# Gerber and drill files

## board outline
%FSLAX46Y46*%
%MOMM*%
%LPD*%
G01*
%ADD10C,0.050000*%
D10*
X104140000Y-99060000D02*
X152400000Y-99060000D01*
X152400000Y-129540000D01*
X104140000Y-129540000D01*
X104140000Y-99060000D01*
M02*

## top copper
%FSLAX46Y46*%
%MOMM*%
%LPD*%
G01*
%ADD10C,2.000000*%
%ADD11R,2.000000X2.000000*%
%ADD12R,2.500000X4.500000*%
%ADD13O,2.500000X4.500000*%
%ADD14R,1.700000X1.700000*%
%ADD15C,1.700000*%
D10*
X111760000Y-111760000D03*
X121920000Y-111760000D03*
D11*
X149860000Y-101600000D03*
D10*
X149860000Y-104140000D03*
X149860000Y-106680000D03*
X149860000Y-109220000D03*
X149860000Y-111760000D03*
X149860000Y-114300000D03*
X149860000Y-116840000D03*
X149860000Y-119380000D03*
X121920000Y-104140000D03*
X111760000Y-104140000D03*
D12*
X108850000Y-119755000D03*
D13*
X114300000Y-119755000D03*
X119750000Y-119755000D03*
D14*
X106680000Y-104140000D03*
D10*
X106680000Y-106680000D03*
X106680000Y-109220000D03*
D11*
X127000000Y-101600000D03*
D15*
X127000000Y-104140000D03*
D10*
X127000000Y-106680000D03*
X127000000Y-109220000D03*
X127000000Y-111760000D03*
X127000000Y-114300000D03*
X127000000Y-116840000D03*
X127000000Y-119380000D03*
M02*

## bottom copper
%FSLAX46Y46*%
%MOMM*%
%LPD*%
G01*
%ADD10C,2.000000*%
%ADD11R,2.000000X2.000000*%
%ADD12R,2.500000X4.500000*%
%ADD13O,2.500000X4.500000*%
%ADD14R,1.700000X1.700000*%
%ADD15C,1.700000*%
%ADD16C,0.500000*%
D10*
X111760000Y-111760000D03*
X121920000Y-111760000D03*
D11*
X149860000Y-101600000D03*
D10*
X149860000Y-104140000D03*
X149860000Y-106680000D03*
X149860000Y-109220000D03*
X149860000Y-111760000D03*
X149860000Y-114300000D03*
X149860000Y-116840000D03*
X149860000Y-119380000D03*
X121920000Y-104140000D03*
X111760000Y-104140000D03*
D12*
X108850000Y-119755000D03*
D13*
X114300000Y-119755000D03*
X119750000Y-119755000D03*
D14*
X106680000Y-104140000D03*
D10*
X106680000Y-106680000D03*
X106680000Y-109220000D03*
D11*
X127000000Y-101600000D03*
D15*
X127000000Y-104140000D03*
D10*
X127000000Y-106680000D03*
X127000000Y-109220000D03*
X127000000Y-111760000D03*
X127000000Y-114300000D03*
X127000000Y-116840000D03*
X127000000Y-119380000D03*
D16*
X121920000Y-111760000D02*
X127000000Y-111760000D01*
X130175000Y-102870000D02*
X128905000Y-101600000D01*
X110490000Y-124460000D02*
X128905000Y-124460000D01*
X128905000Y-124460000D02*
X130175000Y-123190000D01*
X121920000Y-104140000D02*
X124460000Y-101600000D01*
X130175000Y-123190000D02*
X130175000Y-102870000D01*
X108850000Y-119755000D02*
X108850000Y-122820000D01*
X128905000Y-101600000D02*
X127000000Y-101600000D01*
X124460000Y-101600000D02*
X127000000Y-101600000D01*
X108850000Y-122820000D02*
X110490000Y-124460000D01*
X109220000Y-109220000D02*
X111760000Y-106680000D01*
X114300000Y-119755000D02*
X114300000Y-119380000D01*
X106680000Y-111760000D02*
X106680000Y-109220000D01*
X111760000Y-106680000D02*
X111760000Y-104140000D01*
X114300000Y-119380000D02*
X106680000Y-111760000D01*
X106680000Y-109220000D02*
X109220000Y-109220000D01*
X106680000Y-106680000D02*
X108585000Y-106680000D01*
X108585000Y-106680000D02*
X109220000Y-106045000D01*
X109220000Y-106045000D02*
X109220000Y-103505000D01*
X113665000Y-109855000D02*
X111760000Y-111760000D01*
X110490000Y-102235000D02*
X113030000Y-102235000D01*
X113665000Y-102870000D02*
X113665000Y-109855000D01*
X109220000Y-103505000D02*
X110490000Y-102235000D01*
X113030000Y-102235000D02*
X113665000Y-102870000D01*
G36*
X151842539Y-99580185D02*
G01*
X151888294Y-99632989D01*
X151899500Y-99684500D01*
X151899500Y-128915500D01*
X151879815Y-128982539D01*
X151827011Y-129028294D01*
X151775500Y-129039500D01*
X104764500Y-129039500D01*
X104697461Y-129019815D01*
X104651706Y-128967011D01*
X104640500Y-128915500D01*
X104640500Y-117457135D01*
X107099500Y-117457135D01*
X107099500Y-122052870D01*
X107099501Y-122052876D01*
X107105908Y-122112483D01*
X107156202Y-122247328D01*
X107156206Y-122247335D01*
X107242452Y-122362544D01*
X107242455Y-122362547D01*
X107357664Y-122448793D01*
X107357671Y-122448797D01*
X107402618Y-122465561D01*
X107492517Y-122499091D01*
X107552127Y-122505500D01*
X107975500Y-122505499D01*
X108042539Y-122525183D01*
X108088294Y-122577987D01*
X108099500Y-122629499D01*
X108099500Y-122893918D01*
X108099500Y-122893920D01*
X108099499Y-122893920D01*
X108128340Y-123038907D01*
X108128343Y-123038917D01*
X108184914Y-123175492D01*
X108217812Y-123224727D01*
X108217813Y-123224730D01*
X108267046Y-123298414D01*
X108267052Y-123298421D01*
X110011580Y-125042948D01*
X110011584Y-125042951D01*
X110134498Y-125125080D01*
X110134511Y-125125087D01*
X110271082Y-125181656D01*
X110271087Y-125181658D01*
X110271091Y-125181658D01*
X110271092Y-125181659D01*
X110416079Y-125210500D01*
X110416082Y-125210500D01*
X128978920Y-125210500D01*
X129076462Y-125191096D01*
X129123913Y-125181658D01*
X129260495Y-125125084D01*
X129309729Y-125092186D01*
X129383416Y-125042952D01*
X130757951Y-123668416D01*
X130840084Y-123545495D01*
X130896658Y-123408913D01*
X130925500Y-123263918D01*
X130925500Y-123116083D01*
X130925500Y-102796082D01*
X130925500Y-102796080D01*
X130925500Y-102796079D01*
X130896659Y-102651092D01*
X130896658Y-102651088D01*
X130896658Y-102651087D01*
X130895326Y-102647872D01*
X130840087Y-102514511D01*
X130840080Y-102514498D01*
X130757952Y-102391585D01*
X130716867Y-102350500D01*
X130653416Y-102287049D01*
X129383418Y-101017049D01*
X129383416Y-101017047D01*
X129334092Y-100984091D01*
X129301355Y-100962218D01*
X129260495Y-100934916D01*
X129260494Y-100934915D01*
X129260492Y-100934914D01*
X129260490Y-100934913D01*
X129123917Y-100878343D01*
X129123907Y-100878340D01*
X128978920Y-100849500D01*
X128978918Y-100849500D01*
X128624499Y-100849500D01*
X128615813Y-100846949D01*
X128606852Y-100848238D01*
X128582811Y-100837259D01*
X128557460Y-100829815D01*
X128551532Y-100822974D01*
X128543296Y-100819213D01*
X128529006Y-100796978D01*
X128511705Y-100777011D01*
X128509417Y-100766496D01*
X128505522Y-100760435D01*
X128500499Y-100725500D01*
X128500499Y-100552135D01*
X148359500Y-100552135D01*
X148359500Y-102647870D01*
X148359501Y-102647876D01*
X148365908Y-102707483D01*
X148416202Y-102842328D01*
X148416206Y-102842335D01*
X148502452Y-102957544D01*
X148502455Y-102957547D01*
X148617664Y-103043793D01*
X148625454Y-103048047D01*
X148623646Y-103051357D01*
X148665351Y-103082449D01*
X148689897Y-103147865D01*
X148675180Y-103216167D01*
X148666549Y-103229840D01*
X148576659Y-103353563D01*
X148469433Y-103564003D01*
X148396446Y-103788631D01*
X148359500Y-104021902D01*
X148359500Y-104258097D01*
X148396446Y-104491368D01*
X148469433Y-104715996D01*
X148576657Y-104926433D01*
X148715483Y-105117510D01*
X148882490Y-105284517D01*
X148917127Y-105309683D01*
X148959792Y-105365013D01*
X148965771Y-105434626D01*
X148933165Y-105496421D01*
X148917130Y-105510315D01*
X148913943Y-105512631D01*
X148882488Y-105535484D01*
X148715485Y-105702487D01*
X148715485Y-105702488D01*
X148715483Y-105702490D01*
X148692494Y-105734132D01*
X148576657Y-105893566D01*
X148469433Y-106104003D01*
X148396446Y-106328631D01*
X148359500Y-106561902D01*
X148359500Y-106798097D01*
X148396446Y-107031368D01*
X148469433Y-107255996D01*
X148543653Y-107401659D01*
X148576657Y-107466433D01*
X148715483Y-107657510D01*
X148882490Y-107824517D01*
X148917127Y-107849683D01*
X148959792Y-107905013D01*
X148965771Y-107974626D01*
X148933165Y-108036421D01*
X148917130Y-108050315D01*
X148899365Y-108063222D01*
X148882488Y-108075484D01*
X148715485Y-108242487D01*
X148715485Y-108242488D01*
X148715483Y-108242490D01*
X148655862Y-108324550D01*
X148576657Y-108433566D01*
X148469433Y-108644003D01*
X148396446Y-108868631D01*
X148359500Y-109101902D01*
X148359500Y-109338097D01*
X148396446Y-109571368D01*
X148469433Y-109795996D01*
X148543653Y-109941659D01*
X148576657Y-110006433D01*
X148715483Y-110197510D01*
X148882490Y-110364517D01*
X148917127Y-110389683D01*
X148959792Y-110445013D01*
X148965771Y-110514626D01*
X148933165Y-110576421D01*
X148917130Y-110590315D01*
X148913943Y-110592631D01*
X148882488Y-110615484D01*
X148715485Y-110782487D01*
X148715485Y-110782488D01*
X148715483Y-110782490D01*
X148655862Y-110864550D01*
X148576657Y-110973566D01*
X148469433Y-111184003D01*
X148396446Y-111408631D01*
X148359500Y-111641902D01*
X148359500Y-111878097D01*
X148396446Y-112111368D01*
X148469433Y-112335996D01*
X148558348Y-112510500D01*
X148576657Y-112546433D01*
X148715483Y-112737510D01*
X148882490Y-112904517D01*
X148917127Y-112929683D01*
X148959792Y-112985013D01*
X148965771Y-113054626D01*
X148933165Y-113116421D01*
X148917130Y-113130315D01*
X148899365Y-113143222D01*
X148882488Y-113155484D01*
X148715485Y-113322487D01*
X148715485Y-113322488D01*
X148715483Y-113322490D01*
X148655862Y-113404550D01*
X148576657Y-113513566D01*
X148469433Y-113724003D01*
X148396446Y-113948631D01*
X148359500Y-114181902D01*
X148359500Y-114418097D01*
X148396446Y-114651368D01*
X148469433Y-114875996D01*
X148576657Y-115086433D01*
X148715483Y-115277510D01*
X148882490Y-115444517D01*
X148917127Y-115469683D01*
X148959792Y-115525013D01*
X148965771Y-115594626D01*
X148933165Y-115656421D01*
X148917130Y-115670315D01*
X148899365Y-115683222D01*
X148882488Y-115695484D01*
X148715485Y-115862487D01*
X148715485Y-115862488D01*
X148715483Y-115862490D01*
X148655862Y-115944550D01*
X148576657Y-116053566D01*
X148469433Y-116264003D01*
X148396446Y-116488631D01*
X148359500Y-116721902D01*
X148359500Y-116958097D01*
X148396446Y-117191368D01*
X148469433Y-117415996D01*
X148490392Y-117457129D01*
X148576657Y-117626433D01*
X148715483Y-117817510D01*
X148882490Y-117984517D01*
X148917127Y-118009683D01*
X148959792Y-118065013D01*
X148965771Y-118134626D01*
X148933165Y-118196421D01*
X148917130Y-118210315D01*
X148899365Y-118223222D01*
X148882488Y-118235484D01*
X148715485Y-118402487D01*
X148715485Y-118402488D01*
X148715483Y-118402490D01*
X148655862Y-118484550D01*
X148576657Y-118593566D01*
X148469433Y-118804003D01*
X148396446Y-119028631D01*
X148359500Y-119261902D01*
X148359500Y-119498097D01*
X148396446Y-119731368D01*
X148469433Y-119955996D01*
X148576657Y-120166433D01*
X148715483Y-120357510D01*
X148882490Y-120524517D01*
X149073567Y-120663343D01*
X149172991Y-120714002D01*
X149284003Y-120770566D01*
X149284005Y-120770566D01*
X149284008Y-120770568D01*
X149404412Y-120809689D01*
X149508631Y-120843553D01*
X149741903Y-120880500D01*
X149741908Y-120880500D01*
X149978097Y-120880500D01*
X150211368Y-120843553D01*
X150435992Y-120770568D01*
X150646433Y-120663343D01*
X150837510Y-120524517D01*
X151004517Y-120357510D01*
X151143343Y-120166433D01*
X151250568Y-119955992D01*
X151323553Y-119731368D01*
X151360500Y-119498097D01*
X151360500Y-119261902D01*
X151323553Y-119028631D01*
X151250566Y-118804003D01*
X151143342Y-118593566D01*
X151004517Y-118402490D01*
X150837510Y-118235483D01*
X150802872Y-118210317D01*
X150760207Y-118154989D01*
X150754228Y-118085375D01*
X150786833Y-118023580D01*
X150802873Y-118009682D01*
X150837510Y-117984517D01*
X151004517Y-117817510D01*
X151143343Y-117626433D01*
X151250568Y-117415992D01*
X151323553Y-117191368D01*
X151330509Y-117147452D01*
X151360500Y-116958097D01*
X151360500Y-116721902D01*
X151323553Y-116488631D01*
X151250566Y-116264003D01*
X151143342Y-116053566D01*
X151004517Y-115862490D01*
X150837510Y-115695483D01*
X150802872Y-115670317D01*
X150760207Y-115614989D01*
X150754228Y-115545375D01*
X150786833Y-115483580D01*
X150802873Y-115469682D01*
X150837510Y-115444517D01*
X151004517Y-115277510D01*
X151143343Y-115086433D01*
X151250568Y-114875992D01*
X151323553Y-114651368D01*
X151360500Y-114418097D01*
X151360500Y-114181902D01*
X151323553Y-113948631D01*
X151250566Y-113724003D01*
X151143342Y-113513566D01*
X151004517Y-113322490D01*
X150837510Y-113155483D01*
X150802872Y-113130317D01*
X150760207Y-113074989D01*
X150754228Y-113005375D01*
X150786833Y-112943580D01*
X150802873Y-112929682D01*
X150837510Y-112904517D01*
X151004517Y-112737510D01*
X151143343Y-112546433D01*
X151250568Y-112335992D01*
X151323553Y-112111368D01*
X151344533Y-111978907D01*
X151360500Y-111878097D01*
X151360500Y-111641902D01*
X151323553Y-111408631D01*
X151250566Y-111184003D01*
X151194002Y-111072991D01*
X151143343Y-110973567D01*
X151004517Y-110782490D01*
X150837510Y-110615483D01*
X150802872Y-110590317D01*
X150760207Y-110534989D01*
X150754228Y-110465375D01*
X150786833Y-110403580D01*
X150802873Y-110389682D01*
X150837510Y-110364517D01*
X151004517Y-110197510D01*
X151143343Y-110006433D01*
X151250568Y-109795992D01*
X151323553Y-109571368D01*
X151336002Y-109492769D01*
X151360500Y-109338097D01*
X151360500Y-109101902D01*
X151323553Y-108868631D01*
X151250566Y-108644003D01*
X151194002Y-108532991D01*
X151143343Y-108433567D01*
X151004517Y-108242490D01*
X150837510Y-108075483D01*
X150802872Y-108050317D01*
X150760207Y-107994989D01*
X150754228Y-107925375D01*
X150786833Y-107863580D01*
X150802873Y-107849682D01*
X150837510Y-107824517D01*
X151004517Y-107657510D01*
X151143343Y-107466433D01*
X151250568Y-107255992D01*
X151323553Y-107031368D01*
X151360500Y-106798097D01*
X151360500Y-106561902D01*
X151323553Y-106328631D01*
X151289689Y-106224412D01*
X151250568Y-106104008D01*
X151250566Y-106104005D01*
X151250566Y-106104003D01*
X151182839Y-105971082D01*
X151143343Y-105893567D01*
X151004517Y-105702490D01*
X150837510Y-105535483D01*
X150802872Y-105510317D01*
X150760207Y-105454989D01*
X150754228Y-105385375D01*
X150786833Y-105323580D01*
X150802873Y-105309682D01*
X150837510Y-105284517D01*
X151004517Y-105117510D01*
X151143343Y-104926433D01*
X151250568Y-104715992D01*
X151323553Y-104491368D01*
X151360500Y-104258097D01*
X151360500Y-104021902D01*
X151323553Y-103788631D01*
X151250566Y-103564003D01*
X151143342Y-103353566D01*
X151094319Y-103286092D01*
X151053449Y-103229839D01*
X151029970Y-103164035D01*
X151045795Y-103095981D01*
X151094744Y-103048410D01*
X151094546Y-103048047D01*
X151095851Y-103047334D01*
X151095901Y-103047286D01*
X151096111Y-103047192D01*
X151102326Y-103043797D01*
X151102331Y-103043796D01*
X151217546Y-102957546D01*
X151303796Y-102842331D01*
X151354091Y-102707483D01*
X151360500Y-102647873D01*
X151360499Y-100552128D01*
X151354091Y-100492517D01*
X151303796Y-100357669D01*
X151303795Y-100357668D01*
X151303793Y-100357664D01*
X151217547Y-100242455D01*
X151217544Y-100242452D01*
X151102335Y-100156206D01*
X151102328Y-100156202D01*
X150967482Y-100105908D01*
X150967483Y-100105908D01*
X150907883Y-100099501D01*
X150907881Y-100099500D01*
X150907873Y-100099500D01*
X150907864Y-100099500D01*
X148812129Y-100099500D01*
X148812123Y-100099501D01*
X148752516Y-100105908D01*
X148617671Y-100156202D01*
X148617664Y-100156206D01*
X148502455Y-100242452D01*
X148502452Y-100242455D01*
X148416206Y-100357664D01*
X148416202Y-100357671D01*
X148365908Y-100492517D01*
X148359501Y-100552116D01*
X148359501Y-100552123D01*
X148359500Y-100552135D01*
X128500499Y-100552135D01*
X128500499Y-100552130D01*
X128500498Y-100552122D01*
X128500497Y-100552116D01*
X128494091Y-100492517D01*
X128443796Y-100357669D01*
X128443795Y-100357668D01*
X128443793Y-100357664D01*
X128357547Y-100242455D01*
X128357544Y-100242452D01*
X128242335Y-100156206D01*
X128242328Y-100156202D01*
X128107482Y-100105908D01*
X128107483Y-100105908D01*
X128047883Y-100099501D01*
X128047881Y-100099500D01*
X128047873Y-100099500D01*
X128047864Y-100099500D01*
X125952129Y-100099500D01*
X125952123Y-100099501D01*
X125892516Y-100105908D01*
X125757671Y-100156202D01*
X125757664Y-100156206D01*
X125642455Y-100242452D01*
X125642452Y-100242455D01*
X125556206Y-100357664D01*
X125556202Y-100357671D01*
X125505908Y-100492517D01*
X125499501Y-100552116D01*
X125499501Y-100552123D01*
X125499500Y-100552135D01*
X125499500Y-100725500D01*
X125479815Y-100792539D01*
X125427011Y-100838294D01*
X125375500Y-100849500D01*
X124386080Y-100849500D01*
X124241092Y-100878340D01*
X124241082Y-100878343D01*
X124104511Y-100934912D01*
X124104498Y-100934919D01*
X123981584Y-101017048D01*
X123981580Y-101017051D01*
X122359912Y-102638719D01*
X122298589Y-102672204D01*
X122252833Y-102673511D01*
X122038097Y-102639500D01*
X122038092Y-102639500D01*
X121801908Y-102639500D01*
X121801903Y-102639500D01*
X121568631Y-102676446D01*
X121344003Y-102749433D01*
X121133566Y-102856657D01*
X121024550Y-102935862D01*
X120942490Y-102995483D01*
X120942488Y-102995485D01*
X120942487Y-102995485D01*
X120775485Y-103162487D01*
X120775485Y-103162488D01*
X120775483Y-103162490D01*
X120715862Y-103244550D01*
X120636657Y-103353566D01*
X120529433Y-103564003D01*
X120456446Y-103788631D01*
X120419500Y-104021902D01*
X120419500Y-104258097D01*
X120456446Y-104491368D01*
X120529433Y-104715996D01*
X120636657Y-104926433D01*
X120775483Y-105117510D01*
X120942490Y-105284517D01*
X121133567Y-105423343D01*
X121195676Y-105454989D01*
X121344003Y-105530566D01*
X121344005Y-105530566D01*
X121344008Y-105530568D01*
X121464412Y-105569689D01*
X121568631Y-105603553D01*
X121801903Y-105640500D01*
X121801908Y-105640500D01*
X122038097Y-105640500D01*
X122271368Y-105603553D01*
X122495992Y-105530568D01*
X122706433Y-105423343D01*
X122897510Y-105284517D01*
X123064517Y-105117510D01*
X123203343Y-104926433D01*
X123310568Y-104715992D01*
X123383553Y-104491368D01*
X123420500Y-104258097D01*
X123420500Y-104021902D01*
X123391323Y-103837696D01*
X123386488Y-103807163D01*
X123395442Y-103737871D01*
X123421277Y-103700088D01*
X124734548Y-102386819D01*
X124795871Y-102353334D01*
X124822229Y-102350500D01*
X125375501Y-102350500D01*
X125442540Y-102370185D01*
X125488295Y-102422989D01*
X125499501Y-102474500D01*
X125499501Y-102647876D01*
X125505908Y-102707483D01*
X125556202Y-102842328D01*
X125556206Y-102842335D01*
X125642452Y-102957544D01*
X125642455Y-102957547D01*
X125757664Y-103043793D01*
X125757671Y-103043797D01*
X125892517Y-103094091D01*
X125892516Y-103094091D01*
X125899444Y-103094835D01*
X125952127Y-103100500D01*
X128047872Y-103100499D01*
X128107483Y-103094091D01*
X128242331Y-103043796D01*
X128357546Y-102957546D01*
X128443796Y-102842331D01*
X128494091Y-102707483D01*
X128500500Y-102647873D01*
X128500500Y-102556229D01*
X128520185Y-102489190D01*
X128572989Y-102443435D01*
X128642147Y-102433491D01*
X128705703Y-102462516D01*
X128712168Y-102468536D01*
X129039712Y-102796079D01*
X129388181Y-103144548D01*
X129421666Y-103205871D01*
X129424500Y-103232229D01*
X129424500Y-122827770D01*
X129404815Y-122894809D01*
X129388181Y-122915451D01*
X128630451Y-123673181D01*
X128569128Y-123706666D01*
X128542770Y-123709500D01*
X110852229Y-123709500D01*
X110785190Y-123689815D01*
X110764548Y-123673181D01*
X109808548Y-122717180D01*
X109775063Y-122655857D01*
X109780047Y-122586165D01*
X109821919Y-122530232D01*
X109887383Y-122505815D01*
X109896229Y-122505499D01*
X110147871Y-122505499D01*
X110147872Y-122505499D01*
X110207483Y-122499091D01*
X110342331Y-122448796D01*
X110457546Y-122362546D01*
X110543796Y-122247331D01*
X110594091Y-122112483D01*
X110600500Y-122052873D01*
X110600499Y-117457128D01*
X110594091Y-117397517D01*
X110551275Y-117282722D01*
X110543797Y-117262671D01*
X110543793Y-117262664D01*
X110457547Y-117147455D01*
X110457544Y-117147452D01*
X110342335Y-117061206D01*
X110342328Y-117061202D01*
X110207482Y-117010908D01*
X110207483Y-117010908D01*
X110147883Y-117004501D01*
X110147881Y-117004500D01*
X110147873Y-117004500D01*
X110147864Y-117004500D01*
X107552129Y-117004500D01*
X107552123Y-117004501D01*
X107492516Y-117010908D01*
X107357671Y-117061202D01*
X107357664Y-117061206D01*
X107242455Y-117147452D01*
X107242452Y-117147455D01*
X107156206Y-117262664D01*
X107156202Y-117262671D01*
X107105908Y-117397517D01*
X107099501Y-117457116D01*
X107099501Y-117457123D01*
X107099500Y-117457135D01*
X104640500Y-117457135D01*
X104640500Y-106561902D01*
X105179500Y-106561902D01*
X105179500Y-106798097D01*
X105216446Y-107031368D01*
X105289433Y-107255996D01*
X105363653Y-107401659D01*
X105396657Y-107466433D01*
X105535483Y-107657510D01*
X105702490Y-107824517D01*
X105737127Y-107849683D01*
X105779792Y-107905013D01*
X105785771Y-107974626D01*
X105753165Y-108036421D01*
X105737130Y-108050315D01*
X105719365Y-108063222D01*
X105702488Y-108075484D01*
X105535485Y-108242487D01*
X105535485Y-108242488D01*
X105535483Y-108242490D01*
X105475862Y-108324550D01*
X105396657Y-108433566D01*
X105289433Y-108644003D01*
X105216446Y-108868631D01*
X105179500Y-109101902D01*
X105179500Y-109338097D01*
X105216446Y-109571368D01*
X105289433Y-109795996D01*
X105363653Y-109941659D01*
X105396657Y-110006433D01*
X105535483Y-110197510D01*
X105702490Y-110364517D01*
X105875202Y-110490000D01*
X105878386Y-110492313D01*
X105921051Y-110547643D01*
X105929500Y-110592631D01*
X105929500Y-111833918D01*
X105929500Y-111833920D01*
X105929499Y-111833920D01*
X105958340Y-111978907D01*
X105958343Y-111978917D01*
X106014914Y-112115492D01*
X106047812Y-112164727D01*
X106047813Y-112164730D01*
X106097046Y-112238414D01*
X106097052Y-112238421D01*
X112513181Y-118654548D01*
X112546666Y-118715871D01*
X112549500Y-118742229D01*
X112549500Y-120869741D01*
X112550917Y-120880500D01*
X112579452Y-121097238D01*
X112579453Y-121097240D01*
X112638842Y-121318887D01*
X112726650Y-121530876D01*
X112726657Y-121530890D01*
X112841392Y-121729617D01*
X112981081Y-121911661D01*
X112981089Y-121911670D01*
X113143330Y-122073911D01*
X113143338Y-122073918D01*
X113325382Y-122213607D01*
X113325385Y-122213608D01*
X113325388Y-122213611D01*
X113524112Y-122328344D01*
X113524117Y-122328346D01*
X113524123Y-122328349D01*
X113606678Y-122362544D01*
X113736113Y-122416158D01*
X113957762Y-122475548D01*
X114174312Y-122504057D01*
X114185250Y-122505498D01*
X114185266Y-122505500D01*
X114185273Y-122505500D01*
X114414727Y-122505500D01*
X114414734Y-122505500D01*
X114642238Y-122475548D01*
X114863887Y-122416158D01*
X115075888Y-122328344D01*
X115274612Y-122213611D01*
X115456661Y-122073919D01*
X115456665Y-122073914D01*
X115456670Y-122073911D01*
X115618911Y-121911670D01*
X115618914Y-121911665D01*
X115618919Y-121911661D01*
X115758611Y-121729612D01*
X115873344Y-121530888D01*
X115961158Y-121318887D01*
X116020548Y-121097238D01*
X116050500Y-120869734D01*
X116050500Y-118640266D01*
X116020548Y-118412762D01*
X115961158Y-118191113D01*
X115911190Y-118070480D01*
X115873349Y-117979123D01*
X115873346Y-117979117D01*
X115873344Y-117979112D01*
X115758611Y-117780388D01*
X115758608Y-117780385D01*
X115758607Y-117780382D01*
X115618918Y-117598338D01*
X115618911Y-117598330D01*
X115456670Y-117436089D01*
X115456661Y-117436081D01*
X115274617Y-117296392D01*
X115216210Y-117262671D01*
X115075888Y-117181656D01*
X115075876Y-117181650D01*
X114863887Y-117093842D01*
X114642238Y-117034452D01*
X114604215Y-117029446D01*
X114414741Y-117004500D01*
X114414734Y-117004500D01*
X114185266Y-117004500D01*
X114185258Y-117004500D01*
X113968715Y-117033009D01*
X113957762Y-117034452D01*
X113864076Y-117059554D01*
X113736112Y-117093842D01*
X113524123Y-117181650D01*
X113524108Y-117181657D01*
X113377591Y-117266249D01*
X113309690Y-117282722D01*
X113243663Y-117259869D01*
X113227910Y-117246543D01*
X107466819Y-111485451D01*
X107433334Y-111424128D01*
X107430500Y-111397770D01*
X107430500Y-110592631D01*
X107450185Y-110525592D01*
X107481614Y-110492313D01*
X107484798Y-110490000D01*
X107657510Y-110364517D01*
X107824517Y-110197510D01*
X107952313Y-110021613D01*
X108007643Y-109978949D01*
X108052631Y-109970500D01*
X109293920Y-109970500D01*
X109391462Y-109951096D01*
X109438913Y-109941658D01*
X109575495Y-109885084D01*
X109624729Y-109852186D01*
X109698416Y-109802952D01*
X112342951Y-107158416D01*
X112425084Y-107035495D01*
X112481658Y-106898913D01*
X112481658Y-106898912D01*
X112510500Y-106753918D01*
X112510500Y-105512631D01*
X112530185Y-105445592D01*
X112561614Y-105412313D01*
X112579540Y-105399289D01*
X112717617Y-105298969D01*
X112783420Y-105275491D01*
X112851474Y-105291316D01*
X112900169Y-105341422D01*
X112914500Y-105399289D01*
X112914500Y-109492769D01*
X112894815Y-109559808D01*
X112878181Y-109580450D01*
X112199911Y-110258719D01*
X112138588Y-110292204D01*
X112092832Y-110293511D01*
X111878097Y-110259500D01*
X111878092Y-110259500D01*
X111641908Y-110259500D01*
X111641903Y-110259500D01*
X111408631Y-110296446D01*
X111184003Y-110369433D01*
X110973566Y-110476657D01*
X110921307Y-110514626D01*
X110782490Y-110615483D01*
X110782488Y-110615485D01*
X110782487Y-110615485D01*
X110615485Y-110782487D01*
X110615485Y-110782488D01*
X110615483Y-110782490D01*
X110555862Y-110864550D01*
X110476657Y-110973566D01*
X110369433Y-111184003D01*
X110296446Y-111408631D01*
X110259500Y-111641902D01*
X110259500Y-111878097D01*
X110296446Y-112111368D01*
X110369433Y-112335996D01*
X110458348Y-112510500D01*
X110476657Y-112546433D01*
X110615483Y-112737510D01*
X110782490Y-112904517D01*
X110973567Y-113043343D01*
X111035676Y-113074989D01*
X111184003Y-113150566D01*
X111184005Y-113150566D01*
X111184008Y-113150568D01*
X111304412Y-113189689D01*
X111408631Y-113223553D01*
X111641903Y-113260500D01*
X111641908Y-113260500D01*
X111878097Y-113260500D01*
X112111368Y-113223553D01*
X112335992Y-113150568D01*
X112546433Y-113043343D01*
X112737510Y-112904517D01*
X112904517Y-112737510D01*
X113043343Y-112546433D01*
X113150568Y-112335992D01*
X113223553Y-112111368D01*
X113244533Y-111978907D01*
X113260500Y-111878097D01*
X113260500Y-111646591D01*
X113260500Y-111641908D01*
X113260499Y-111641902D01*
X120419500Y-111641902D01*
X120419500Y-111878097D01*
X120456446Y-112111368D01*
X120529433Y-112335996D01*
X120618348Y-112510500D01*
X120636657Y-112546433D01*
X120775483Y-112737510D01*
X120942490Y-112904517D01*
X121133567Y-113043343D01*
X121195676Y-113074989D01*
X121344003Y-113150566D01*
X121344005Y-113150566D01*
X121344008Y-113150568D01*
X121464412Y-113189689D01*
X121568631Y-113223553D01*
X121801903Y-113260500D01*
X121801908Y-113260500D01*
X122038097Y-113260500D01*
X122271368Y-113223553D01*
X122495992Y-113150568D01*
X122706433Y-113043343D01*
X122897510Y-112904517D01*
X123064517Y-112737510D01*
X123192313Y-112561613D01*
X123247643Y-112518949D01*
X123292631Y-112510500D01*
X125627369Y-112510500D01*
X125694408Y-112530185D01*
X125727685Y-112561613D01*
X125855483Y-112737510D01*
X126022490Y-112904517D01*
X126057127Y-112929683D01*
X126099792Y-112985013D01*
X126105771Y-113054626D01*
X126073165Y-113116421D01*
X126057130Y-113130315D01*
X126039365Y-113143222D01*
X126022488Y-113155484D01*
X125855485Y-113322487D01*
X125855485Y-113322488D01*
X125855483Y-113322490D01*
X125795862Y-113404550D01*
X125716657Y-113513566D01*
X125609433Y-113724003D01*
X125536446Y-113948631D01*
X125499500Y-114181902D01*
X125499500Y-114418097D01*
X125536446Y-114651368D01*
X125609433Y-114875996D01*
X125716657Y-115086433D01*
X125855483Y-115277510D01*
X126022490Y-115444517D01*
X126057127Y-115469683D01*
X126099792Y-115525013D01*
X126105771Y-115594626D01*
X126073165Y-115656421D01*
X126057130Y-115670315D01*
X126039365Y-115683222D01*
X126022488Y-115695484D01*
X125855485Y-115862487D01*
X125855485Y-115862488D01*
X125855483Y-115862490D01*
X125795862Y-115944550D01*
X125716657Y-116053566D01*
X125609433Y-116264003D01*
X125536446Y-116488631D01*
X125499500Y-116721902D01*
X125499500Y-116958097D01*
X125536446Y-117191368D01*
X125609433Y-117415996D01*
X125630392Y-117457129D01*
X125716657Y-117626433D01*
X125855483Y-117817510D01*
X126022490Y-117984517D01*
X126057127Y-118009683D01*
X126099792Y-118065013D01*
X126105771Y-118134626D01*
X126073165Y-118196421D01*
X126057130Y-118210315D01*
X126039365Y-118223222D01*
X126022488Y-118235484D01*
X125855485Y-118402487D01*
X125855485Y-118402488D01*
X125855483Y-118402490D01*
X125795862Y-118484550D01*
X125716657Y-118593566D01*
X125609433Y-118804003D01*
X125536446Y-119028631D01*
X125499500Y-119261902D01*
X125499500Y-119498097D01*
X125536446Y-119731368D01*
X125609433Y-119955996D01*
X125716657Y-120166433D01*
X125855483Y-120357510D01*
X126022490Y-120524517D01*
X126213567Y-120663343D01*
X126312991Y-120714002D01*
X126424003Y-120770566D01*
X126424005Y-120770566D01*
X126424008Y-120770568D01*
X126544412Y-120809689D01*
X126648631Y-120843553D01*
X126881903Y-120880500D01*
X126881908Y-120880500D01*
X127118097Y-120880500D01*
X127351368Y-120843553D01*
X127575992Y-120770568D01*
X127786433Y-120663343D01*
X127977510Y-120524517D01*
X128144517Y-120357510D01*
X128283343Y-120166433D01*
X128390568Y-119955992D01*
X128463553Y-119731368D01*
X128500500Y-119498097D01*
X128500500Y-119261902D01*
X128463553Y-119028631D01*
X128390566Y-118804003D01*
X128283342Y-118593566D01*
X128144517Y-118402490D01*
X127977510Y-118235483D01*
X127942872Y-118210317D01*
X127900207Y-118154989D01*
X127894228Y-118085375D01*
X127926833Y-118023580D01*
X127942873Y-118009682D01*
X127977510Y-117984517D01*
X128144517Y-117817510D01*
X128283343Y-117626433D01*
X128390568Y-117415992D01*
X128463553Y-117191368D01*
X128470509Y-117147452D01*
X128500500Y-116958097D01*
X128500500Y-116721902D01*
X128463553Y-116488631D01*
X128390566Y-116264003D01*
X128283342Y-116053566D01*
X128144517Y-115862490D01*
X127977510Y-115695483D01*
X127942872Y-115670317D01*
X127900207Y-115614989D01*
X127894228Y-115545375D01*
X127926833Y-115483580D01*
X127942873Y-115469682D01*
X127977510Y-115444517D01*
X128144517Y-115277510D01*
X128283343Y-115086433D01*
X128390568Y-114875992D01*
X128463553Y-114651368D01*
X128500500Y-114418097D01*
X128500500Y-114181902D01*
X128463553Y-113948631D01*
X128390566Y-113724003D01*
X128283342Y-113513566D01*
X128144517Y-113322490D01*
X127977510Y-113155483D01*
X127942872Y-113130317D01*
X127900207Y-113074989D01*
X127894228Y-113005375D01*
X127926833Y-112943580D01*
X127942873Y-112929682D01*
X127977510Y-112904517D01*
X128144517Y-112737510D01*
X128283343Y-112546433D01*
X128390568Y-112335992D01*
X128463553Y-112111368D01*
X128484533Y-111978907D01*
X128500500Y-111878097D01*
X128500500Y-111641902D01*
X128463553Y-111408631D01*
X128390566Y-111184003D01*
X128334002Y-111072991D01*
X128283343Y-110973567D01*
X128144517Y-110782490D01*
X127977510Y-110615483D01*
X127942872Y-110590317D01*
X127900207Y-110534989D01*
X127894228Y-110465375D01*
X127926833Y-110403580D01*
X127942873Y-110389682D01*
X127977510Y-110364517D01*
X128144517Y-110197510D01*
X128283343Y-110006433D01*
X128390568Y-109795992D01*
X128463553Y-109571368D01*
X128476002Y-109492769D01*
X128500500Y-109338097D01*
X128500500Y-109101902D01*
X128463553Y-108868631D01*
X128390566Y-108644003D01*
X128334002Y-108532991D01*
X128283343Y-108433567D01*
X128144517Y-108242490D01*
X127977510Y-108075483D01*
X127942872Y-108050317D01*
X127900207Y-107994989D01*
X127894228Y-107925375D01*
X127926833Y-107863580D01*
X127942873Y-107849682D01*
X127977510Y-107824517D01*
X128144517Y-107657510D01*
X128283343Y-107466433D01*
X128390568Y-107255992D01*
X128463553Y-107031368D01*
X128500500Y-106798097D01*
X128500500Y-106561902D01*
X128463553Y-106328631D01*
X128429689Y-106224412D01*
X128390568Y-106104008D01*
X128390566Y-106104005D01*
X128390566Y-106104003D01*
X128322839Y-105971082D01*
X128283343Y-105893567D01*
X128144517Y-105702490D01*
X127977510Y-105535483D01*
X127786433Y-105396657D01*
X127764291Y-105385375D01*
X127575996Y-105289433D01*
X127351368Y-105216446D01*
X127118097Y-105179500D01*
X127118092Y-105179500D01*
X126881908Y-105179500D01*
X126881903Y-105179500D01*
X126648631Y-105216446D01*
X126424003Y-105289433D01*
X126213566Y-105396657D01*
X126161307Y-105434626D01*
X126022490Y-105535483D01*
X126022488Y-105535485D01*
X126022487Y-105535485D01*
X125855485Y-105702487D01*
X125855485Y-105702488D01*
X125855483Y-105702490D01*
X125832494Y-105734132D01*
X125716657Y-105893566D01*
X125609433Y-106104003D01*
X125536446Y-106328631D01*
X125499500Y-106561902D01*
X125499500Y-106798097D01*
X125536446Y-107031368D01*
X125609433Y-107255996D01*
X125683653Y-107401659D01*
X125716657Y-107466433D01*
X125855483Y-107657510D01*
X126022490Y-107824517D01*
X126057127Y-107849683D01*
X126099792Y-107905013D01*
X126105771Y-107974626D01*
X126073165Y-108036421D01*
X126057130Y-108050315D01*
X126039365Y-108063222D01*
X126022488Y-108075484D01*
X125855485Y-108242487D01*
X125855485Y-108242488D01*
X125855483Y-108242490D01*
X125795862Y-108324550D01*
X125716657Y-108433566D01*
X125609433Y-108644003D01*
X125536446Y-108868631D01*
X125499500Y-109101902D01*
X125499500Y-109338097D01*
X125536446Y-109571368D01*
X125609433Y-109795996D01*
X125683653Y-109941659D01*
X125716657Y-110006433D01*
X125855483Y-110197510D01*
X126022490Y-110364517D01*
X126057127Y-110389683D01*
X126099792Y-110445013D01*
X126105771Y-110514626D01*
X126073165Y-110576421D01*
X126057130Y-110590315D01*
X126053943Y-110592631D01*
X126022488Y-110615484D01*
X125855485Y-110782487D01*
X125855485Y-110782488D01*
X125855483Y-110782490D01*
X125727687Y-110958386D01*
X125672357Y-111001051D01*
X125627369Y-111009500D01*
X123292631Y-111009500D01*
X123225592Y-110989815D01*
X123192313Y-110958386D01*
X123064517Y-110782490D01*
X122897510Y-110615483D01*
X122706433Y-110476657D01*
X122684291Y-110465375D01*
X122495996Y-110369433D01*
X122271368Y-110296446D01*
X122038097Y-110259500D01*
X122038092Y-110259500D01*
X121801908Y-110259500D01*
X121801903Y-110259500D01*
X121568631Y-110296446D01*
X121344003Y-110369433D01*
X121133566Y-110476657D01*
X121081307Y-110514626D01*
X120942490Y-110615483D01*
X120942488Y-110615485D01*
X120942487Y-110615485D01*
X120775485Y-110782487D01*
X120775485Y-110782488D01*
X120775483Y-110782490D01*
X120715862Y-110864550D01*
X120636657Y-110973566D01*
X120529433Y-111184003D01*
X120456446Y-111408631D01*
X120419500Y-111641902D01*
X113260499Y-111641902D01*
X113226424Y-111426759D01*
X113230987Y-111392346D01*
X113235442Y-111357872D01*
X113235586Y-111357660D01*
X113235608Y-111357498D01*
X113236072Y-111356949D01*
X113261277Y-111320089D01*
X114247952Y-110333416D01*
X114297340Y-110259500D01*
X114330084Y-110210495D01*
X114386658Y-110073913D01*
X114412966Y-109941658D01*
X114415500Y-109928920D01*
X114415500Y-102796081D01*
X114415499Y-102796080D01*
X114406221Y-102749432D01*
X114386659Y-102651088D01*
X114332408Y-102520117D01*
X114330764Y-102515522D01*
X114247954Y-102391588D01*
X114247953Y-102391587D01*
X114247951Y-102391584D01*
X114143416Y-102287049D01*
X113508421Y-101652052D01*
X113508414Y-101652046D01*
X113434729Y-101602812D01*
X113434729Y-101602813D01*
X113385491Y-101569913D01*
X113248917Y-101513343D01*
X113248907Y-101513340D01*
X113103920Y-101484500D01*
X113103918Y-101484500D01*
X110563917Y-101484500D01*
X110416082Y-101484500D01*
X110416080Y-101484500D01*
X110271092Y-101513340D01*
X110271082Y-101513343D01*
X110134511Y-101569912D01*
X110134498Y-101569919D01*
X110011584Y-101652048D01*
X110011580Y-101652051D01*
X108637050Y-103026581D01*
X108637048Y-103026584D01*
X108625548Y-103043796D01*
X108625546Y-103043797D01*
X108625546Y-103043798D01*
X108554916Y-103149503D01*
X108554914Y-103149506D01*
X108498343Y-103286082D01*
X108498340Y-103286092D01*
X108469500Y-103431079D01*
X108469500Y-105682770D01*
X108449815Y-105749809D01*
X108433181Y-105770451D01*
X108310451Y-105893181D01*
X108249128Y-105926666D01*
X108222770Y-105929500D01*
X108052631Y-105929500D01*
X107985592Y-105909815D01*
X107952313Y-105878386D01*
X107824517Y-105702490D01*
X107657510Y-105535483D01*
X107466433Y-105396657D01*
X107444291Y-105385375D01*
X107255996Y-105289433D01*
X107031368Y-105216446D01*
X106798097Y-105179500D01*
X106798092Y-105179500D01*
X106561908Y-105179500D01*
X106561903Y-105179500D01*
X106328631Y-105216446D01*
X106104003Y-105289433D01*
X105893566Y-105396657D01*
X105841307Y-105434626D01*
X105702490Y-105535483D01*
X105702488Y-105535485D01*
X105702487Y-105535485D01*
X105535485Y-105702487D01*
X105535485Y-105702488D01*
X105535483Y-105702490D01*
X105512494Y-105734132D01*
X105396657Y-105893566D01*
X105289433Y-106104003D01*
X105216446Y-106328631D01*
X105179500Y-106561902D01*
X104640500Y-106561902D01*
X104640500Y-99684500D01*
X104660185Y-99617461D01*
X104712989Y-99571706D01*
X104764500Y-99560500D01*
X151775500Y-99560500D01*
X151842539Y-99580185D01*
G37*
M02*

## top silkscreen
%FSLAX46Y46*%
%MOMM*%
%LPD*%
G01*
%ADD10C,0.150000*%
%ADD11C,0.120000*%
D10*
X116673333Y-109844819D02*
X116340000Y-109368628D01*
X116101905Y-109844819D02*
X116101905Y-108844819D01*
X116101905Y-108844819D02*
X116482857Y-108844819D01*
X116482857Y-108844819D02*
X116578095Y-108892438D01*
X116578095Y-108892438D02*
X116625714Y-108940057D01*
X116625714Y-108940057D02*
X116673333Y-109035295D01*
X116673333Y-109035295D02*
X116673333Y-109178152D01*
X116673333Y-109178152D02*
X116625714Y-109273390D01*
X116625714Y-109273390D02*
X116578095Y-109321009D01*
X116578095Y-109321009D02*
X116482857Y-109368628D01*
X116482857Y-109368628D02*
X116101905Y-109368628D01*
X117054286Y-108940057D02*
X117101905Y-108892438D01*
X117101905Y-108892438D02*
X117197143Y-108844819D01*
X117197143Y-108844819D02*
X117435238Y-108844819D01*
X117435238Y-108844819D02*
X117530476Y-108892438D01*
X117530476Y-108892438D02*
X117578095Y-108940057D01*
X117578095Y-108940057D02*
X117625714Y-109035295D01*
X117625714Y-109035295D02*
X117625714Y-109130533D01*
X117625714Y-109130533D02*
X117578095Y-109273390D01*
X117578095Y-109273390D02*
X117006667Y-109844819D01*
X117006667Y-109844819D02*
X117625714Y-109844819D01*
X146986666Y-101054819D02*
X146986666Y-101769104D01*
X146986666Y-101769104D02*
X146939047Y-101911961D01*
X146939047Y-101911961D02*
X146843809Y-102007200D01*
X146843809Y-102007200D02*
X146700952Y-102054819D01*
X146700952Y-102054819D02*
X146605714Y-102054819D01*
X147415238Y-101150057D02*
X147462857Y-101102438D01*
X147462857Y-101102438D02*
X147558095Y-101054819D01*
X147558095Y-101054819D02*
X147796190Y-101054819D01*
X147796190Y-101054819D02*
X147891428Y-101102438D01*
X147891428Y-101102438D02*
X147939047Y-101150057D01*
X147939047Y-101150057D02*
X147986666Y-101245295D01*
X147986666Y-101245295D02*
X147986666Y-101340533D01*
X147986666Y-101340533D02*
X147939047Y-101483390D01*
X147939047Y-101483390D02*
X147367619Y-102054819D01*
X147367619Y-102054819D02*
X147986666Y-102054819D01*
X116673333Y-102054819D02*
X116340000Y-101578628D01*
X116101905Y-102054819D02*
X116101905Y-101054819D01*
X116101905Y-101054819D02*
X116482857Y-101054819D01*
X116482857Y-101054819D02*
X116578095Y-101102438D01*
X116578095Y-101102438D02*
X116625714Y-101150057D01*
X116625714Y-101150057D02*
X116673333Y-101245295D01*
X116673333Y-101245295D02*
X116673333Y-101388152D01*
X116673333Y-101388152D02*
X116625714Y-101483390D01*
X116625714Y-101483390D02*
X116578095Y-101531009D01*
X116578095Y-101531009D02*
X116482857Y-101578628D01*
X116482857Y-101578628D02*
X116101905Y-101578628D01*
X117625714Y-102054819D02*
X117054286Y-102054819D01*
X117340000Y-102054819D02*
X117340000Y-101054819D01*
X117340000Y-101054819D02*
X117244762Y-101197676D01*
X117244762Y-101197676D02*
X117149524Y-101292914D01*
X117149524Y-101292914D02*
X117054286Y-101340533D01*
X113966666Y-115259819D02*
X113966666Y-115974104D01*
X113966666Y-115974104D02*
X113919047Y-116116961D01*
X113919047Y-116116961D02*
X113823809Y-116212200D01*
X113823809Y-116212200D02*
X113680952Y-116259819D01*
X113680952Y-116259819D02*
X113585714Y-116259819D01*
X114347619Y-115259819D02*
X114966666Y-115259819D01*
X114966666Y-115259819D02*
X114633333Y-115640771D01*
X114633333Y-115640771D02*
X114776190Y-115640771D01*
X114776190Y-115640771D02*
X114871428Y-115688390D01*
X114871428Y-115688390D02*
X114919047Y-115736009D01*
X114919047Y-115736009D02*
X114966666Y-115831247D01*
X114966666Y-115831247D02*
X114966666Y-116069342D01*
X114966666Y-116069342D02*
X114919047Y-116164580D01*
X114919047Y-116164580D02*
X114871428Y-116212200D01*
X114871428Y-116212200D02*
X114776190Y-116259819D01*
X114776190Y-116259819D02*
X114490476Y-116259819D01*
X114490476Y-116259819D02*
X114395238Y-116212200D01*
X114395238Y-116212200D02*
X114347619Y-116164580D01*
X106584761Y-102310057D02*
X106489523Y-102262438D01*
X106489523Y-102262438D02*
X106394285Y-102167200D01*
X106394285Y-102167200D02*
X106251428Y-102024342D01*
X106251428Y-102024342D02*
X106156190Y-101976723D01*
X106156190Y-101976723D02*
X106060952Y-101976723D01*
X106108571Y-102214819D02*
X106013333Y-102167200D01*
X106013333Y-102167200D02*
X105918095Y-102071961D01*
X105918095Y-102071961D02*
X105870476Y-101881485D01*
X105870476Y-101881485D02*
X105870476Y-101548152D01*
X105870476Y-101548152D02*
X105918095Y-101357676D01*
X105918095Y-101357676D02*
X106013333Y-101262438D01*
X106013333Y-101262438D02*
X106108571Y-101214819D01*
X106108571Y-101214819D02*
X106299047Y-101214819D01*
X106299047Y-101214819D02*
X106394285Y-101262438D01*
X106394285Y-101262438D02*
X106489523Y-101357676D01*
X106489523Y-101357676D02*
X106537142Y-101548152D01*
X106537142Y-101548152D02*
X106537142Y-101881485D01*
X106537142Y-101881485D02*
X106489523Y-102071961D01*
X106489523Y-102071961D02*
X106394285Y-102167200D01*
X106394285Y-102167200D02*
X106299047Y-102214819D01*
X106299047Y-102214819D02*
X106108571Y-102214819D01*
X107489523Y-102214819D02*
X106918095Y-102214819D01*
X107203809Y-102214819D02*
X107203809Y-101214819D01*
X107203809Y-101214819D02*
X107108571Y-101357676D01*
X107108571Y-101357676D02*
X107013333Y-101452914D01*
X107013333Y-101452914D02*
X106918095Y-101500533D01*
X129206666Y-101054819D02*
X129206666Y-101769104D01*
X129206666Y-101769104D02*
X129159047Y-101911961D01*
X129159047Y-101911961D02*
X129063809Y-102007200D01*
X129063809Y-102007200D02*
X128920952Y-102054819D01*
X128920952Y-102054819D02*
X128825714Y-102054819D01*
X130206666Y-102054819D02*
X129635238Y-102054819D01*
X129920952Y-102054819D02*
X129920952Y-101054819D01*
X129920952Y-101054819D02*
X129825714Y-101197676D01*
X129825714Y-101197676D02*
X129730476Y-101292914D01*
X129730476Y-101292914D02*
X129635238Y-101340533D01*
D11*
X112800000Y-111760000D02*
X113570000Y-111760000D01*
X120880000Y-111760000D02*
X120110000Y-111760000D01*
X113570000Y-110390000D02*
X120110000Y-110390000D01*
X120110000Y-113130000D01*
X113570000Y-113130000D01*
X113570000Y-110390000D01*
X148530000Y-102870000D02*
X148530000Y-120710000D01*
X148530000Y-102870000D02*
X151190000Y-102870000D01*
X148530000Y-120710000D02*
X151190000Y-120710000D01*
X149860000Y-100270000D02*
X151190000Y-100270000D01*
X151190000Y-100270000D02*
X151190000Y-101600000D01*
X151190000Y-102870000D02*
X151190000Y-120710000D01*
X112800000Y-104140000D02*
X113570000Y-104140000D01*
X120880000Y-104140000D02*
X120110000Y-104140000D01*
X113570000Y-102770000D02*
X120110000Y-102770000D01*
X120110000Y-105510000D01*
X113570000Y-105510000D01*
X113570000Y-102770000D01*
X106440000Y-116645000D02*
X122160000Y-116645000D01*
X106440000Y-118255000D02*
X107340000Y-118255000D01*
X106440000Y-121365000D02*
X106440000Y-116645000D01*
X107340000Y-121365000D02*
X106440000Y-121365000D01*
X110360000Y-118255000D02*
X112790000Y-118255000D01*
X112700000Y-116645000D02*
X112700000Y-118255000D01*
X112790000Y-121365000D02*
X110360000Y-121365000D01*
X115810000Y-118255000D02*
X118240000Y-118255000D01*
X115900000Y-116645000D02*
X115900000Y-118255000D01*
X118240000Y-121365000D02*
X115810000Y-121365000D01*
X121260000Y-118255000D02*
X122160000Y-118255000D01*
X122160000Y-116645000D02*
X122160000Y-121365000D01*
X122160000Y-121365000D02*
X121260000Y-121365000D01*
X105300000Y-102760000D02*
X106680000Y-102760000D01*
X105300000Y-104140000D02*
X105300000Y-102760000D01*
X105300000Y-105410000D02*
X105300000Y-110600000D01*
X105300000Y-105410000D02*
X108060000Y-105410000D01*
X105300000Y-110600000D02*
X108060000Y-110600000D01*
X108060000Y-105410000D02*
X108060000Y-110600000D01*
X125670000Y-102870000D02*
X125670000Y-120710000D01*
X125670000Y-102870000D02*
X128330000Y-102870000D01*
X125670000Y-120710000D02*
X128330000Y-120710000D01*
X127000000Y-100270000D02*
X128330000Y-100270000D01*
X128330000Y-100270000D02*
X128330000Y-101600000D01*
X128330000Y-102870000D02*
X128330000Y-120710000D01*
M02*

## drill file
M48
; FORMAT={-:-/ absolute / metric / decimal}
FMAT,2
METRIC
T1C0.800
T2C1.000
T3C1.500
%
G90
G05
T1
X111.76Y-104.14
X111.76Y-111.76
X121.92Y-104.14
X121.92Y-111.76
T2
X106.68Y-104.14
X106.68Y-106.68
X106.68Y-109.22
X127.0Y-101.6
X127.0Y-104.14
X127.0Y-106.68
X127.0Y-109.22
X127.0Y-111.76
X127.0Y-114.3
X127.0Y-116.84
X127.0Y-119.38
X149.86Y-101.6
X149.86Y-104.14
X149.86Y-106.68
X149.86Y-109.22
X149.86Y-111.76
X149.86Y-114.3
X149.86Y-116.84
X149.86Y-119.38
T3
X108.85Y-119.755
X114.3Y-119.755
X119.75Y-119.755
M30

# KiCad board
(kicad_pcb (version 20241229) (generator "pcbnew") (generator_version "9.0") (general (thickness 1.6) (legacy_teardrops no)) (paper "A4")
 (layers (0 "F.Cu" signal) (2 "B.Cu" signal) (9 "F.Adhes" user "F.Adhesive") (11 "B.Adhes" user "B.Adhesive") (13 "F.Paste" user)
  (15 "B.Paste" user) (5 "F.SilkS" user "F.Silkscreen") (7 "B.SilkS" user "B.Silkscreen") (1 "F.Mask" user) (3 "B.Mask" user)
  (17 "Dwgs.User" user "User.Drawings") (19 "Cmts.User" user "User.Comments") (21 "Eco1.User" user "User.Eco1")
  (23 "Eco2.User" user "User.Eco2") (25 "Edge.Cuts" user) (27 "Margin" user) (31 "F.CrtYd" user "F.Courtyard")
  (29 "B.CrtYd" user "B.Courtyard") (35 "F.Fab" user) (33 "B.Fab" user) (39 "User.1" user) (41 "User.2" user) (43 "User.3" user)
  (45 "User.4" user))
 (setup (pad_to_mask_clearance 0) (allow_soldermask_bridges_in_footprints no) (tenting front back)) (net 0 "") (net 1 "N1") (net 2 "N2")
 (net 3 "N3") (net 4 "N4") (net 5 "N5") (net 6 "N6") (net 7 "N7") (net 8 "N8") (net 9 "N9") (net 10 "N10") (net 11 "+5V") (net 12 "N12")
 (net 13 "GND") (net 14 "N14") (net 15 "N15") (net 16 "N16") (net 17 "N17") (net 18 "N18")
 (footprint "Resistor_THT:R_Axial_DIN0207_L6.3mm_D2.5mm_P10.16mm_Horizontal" (layer "F.Cu") (at 111.76 111.76)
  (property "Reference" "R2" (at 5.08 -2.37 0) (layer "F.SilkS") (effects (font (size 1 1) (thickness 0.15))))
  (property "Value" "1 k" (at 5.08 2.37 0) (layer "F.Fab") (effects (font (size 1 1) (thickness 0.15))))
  (fp_line (start 1.04 0) (end 1.81 0) (stroke (width 0.12) (type solid)) (layer "F.SilkS"))
  (fp_line (start 9.12 0) (end 8.35 0) (stroke (width 0.12) (type solid)) (layer "F.SilkS"))
  (fp_rect (start 1.81 -1.37) (end 8.35 1.37) (stroke (width 0.12) (type solid)) (fill no) (layer "F.SilkS"))
  (pad "1" thru_hole circle (at 0 0) (size 2 2) (drill 0.8) (layers "*.Cu" "*.Mask") (remove_unused_layers no) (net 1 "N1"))
  (pad "2" thru_hole circle (at 10.16 0) (size 2 2) (drill 0.8) (layers "*.Cu" "*.Mask") (remove_unused_layers no) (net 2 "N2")))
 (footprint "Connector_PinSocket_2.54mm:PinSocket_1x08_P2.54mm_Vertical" (layer "F.Cu") (at 149.86 101.6)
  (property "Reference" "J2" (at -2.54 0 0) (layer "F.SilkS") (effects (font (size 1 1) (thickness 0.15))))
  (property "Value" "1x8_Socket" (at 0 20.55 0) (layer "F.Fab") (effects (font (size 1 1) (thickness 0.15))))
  (fp_line (start -1.33 1.27) (end -1.33 19.11) (stroke (width 0.12) (type solid)) (layer "F.SilkS"))
  (fp_line (start -1.33 1.27) (end 1.33 1.27) (stroke (width 0.12) (type solid)) (layer "F.SilkS"))
  (fp_line (start -1.33 19.11) (end 1.33 19.11) (stroke (width 0.12) (type solid)) (layer "F.SilkS"))
  (fp_line (start 0 -1.33) (end 1.33 -1.33) (stroke (width 0.12) (type solid)) (layer "F.SilkS"))
  (fp_line (start 1.33 -1.33) (end 1.33 0) (stroke (width 0.12) (type solid)) (layer "F.SilkS"))
  (fp_line (start 1.33 1.27) (end 1.33 19.11) (stroke (width 0.12) (type solid)) (layer "F.SilkS"))
  (pad "1" thru_hole rect (at 0 0) (size 2 2) (drill 1) (layers "*.Cu" "*.Mask") (remove_unused_layers no) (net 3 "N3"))
  (pad "2" thru_hole circle (at 0 2.54) (size 2 2) (drill 1) (layers "*.Cu" "*.Mask") (remove_unused_layers no) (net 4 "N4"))
  (pad "3" thru_hole circle (at 0 5.08) (size 2 2) (drill 1) (layers "*.Cu" "*.Mask") (remove_unused_layers no) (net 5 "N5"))
  (pad "4" thru_hole circle (at 0 7.62) (size 2 2) (drill 1) (layers "*.Cu" "*.Mask") (remove_unused_layers no) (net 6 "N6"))
  (pad "5" thru_hole circle (at 0 10.16) (size 2 2) (drill 1) (layers "*.Cu" "*.Mask") (remove_unused_layers no) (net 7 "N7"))
  (pad "6" thru_hole circle (at 0 12.7) (size 2 2) (drill 1) (layers "*.Cu" "*.Mask") (remove_unused_layers no) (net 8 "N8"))
  (pad "7" thru_hole circle (at 0 15.24) (size 2 2) (drill 1) (layers "*.Cu" "*.Mask") (remove_unused_layers no) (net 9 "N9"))
  (pad "8" thru_hole circle (at 0 17.78) (size 2 2) (drill 1) (layers "*.Cu" "*.Mask") (remove_unused_layers no) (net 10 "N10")))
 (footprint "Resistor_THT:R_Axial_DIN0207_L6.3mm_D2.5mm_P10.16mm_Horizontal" (layer "F.Cu") (at 121.92 104.14 180)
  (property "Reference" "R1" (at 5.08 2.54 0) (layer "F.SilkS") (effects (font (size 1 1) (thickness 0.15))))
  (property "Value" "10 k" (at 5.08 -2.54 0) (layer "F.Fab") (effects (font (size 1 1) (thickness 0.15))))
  (fp_line (start 9.12 0) (end 8.35 0) (stroke (width 0.12) (type solid)) (layer "F.SilkS"))
  (fp_line (start 1.04 0) (end 1.81 0) (stroke (width 0.12) (type solid)) (layer "F.SilkS"))
  (fp_rect (start 1.81 -1.37) (end 8.35 1.37) (stroke (width 0.12) (type solid)) (fill no) (layer "F.SilkS"))
  (pad "1" thru_hole circle (at 0 0 180) (size 2 2) (drill 0.8) (layers "*.Cu" "*.Mask") (remove_unused_layers no) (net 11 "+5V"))
  (pad "2" thru_hole circle (at 10.16 0 180) (size 2 2) (drill 0.8) (layers "*.Cu" "*.Mask") (remove_unused_layers no) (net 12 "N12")))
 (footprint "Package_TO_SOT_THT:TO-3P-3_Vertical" (layer "F.Cu") (at 108.85 119.755)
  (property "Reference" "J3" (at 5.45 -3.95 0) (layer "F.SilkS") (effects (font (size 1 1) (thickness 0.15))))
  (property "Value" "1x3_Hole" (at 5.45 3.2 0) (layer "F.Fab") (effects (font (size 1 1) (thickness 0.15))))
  (fp_line (start -2.41 -3.11) (end 13.31 -3.11) (stroke (width 0.12) (type solid)) (layer "F.SilkS"))
  (fp_line (start -2.41 -1.5) (end -1.51 -1.5) (stroke (width 0.12) (type solid)) (layer "F.SilkS"))
  (fp_line (start -2.41 1.61) (end -2.41 -3.11) (stroke (width 0.12) (type solid)) (layer "F.SilkS"))
  (fp_line (start -1.51 1.61) (end -2.41 1.61) (stroke (width 0.12) (type solid)) (layer "F.SilkS"))
  (fp_line (start 1.51 -1.5) (end 3.94 -1.5) (stroke (width 0.12) (type solid)) (layer "F.SilkS"))
  (fp_line (start 3.85 -3.11) (end 3.85 -1.5) (stroke (width 0.12) (type solid)) (layer "F.SilkS"))
  (fp_line (start 3.94 1.61) (end 1.51 1.61) (stroke (width 0.12) (type solid)) (layer "F.SilkS"))
  (fp_line (start 6.96 -1.5) (end 9.39 -1.5) (stroke (width 0.12) (type solid)) (layer "F.SilkS"))
  (fp_line (start 7.05 -3.11) (end 7.05 -1.5) (stroke (width 0.12) (type solid)) (layer "F.SilkS"))
  (fp_line (start 9.39 1.61) (end 6.96 1.61) (stroke (width 0.12) (type solid)) (layer "F.SilkS"))
  (fp_line (start 12.41 -1.5) (end 13.31 -1.5) (stroke (width 0.12) (type solid)) (layer "F.SilkS"))
  (fp_line (start 13.31 -3.11) (end 13.31 1.61) (stroke (width 0.12) (type solid)) (layer "F.SilkS"))
  (fp_line (start 13.31 1.61) (end 12.41 1.61) (stroke (width 0.12) (type solid)) (layer "F.SilkS"))
  (pad "1" thru_hole rect (at 0 0) (size 2.5 4.5) (drill 1.5) (layers "*.Cu" "*.Mask") (remove_unused_layers no) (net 11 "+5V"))
  (pad "2" thru_hole oval (at 5.45 0) (size 2.5 4.5) (drill 1.5) (layers "*.Cu" "*.Mask") (remove_unused_layers no) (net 12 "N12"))
  (pad "3" thru_hole oval (at 10.9 0) (size 2.5 4.5) (drill 1.5) (layers "*.Cu" "*.Mask") (remove_unused_layers no) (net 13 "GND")))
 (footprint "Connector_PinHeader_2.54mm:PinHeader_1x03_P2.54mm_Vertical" (layer "F.Cu") (at 106.68 104.14)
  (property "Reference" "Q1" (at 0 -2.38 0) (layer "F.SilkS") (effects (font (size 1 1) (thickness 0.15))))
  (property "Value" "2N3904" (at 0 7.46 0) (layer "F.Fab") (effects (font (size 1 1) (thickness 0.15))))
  (fp_line (start -1.38 -1.38) (end 0 -1.38) (stroke (width 0.12) (type solid)) (layer "F.SilkS"))
  (fp_line (start -1.38 0) (end -1.38 -1.38) (stroke (width 0.12) (type solid)) (layer "F.SilkS"))
  (fp_line (start -1.38 1.27) (end -1.38 6.46) (stroke (width 0.12) (type solid)) (layer "F.SilkS"))
  (fp_line (start -1.38 1.27) (end 1.38 1.27) (stroke (width 0.12) (type solid)) (layer "F.SilkS"))
  (fp_line (start -1.38 6.46) (end 1.38 6.46) (stroke (width 0.12) (type solid)) (layer "F.SilkS"))
  (fp_line (start 1.38 1.27) (end 1.38 6.46) (stroke (width 0.12) (type solid)) (layer "F.SilkS"))
  (pad "1" thru_hole rect (at 0 0) (size 1.7 1.7) (drill 1) (layers "*.Cu" "*.Mask") (remove_unused_layers no) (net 13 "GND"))
  (pad "2" thru_hole circle (at 0 2.54) (size 2 2) (drill 1) (layers "*.Cu" "*.Mask") (remove_unused_layers no) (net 1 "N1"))
  (pad "3" thru_hole circle (at 0 5.08) (size 2 2) (drill 1) (layers "*.Cu" "*.Mask") (remove_unused_layers no) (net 12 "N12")))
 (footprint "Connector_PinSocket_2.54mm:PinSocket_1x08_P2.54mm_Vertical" (layer "F.Cu") (at 127 101.6)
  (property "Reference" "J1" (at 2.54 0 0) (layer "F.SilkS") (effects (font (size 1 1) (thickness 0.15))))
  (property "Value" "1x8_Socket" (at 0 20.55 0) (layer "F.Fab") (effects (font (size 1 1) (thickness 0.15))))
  (fp_line (start -1.33 1.27) (end -1.33 19.11) (stroke (width 0.12) (type solid)) (layer "F.SilkS"))
  (fp_line (start -1.33 1.27) (end 1.33 1.27) (stroke (width 0.12) (type solid)) (layer "F.SilkS"))
  (fp_line (start -1.33 19.11) (end 1.33 19.11) (stroke (width 0.12) (type solid)) (layer "F.SilkS"))
  (fp_line (start 0 -1.33) (end 1.33 -1.33) (stroke (width 0.12) (type solid)) (layer "F.SilkS"))
  (fp_line (start 1.33 -1.33) (end 1.33 0) (stroke (width 0.12) (type solid)) (layer "F.SilkS"))
  (fp_line (start 1.33 1.27) (end 1.33 19.11) (stroke (width 0.12) (type solid)) (layer "F.SilkS"))
  (pad "1" thru_hole rect (at 0 0) (size 2 2) (drill 1) (layers "*.Cu" "*.Mask") (remove_unused_layers no) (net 11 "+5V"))
  (pad "2" thru_hole circle (at 0 2.54) (size 1.7 1.7) (drill 1) (layers "*.Cu" "*.Mask") (remove_unused_layers no) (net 13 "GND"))
  (pad "3" thru_hole circle (at 0 5.08) (size 2 2) (drill 1) (layers "*.Cu" "*.Mask") (remove_unused_layers no) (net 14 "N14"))
  (pad "4" thru_hole circle (at 0 7.62) (size 2 2) (drill 1) (layers "*.Cu" "*.Mask") (remove_unused_layers no) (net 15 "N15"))
  (pad "5" thru_hole circle (at 0 10.16) (size 2 2) (drill 1) (layers "*.Cu" "*.Mask") (remove_unused_layers no) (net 2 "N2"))
  (pad "6" thru_hole circle (at 0 12.7) (size 2 2) (drill 1) (layers "*.Cu" "*.Mask") (remove_unused_layers no) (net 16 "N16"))
  (pad "7" thru_hole circle (at 0 15.24) (size 2 2) (drill 1) (layers "*.Cu" "*.Mask") (remove_unused_layers no) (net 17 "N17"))
  (pad "8" thru_hole circle (at 0 17.78) (size 2 2) (drill 1) (layers "*.Cu" "*.Mask") (remove_unused_layers no) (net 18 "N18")))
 (gr_rect (start 104.14 99.06) (end 152.4 129.54) (stroke (width 0.05) (type default)) (fill no) (layer "Edge.Cuts"))
 (segment (start 121.92 111.76) (end 127 111.76) (width 0.5) (layer "B.Cu") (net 2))
 (segment (start 130.175 102.87) (end 128.905 101.6) (width 0.5) (layer "B.Cu") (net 11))
 (segment (start 110.49 124.46) (end 128.905 124.46) (width 0.5) (layer "B.Cu") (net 11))
 (segment (start 128.905 124.46) (end 130.175 123.19) (width 0.5) (layer "B.Cu") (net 11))
 (segment (start 121.92 104.14) (end 124.46 101.6) (width 0.5) (layer "B.Cu") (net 11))
 (segment (start 130.175 123.19) (end 130.175 102.87) (width 0.5) (layer "B.Cu") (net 11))
 (segment (start 108.85 119.755) (end 108.85 122.82) (width 0.5) (layer "B.Cu") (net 11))
 (segment (start 128.905 101.6) (end 127 101.6) (width 0.5) (layer "B.Cu") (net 11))
 (segment (start 124.46 101.6) (end 127 101.6) (width 0.5) (layer "B.Cu") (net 11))
 (segment (start 108.85 122.82) (end 110.49 124.46) (width 0.5) (layer "B.Cu") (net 11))
 (segment (start 109.22 109.22) (end 111.76 106.68) (width 0.5) (layer "B.Cu") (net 12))
 (segment (start 114.3 119.755) (end 114.3 119.38) (width 0.5) (layer "B.Cu") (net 12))
 (segment (start 106.68 111.76) (end 106.68 109.22) (width 0.5) (layer "B.Cu") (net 12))
 (segment (start 111.76 106.68) (end 111.76 104.14) (width 0.5) (layer "B.Cu") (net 12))
 (segment (start 114.3 119.38) (end 106.68 111.76) (width 0.5) (layer "B.Cu") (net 12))
 (segment (start 106.68 109.22) (end 109.22 109.22) (width 0.5) (layer "B.Cu") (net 12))
 (segment (start 106.68 106.68) (end 108.585 106.68) (width 0.5) (layer "B.Cu") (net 1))
 (segment (start 108.585 106.68) (end 109.22 106.045) (width 0.5) (layer "B.Cu") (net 1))
 (segment (start 109.22 106.045) (end 109.22 103.505) (width 0.5) (layer "B.Cu") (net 1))
 (segment (start 113.665 109.855) (end 111.76 111.76) (width 0.5) (layer "B.Cu") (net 1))
 (segment (start 110.49 102.235) (end 113.03 102.235) (width 0.5) (layer "B.Cu") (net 1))
 (segment (start 113.665 102.87) (end 113.665 109.855) (width 0.5) (layer "B.Cu") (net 1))
 (segment (start 109.22 103.505) (end 110.49 102.235) (width 0.5) (layer "B.Cu") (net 1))
 (segment (start 113.03 102.235) (end 113.665 102.87) (width 0.5) (layer "B.Cu") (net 1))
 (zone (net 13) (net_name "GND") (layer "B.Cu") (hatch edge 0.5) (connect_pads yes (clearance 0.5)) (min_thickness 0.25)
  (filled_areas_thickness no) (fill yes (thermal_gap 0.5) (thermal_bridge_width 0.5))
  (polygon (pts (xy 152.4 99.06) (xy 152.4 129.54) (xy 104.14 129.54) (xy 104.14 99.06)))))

